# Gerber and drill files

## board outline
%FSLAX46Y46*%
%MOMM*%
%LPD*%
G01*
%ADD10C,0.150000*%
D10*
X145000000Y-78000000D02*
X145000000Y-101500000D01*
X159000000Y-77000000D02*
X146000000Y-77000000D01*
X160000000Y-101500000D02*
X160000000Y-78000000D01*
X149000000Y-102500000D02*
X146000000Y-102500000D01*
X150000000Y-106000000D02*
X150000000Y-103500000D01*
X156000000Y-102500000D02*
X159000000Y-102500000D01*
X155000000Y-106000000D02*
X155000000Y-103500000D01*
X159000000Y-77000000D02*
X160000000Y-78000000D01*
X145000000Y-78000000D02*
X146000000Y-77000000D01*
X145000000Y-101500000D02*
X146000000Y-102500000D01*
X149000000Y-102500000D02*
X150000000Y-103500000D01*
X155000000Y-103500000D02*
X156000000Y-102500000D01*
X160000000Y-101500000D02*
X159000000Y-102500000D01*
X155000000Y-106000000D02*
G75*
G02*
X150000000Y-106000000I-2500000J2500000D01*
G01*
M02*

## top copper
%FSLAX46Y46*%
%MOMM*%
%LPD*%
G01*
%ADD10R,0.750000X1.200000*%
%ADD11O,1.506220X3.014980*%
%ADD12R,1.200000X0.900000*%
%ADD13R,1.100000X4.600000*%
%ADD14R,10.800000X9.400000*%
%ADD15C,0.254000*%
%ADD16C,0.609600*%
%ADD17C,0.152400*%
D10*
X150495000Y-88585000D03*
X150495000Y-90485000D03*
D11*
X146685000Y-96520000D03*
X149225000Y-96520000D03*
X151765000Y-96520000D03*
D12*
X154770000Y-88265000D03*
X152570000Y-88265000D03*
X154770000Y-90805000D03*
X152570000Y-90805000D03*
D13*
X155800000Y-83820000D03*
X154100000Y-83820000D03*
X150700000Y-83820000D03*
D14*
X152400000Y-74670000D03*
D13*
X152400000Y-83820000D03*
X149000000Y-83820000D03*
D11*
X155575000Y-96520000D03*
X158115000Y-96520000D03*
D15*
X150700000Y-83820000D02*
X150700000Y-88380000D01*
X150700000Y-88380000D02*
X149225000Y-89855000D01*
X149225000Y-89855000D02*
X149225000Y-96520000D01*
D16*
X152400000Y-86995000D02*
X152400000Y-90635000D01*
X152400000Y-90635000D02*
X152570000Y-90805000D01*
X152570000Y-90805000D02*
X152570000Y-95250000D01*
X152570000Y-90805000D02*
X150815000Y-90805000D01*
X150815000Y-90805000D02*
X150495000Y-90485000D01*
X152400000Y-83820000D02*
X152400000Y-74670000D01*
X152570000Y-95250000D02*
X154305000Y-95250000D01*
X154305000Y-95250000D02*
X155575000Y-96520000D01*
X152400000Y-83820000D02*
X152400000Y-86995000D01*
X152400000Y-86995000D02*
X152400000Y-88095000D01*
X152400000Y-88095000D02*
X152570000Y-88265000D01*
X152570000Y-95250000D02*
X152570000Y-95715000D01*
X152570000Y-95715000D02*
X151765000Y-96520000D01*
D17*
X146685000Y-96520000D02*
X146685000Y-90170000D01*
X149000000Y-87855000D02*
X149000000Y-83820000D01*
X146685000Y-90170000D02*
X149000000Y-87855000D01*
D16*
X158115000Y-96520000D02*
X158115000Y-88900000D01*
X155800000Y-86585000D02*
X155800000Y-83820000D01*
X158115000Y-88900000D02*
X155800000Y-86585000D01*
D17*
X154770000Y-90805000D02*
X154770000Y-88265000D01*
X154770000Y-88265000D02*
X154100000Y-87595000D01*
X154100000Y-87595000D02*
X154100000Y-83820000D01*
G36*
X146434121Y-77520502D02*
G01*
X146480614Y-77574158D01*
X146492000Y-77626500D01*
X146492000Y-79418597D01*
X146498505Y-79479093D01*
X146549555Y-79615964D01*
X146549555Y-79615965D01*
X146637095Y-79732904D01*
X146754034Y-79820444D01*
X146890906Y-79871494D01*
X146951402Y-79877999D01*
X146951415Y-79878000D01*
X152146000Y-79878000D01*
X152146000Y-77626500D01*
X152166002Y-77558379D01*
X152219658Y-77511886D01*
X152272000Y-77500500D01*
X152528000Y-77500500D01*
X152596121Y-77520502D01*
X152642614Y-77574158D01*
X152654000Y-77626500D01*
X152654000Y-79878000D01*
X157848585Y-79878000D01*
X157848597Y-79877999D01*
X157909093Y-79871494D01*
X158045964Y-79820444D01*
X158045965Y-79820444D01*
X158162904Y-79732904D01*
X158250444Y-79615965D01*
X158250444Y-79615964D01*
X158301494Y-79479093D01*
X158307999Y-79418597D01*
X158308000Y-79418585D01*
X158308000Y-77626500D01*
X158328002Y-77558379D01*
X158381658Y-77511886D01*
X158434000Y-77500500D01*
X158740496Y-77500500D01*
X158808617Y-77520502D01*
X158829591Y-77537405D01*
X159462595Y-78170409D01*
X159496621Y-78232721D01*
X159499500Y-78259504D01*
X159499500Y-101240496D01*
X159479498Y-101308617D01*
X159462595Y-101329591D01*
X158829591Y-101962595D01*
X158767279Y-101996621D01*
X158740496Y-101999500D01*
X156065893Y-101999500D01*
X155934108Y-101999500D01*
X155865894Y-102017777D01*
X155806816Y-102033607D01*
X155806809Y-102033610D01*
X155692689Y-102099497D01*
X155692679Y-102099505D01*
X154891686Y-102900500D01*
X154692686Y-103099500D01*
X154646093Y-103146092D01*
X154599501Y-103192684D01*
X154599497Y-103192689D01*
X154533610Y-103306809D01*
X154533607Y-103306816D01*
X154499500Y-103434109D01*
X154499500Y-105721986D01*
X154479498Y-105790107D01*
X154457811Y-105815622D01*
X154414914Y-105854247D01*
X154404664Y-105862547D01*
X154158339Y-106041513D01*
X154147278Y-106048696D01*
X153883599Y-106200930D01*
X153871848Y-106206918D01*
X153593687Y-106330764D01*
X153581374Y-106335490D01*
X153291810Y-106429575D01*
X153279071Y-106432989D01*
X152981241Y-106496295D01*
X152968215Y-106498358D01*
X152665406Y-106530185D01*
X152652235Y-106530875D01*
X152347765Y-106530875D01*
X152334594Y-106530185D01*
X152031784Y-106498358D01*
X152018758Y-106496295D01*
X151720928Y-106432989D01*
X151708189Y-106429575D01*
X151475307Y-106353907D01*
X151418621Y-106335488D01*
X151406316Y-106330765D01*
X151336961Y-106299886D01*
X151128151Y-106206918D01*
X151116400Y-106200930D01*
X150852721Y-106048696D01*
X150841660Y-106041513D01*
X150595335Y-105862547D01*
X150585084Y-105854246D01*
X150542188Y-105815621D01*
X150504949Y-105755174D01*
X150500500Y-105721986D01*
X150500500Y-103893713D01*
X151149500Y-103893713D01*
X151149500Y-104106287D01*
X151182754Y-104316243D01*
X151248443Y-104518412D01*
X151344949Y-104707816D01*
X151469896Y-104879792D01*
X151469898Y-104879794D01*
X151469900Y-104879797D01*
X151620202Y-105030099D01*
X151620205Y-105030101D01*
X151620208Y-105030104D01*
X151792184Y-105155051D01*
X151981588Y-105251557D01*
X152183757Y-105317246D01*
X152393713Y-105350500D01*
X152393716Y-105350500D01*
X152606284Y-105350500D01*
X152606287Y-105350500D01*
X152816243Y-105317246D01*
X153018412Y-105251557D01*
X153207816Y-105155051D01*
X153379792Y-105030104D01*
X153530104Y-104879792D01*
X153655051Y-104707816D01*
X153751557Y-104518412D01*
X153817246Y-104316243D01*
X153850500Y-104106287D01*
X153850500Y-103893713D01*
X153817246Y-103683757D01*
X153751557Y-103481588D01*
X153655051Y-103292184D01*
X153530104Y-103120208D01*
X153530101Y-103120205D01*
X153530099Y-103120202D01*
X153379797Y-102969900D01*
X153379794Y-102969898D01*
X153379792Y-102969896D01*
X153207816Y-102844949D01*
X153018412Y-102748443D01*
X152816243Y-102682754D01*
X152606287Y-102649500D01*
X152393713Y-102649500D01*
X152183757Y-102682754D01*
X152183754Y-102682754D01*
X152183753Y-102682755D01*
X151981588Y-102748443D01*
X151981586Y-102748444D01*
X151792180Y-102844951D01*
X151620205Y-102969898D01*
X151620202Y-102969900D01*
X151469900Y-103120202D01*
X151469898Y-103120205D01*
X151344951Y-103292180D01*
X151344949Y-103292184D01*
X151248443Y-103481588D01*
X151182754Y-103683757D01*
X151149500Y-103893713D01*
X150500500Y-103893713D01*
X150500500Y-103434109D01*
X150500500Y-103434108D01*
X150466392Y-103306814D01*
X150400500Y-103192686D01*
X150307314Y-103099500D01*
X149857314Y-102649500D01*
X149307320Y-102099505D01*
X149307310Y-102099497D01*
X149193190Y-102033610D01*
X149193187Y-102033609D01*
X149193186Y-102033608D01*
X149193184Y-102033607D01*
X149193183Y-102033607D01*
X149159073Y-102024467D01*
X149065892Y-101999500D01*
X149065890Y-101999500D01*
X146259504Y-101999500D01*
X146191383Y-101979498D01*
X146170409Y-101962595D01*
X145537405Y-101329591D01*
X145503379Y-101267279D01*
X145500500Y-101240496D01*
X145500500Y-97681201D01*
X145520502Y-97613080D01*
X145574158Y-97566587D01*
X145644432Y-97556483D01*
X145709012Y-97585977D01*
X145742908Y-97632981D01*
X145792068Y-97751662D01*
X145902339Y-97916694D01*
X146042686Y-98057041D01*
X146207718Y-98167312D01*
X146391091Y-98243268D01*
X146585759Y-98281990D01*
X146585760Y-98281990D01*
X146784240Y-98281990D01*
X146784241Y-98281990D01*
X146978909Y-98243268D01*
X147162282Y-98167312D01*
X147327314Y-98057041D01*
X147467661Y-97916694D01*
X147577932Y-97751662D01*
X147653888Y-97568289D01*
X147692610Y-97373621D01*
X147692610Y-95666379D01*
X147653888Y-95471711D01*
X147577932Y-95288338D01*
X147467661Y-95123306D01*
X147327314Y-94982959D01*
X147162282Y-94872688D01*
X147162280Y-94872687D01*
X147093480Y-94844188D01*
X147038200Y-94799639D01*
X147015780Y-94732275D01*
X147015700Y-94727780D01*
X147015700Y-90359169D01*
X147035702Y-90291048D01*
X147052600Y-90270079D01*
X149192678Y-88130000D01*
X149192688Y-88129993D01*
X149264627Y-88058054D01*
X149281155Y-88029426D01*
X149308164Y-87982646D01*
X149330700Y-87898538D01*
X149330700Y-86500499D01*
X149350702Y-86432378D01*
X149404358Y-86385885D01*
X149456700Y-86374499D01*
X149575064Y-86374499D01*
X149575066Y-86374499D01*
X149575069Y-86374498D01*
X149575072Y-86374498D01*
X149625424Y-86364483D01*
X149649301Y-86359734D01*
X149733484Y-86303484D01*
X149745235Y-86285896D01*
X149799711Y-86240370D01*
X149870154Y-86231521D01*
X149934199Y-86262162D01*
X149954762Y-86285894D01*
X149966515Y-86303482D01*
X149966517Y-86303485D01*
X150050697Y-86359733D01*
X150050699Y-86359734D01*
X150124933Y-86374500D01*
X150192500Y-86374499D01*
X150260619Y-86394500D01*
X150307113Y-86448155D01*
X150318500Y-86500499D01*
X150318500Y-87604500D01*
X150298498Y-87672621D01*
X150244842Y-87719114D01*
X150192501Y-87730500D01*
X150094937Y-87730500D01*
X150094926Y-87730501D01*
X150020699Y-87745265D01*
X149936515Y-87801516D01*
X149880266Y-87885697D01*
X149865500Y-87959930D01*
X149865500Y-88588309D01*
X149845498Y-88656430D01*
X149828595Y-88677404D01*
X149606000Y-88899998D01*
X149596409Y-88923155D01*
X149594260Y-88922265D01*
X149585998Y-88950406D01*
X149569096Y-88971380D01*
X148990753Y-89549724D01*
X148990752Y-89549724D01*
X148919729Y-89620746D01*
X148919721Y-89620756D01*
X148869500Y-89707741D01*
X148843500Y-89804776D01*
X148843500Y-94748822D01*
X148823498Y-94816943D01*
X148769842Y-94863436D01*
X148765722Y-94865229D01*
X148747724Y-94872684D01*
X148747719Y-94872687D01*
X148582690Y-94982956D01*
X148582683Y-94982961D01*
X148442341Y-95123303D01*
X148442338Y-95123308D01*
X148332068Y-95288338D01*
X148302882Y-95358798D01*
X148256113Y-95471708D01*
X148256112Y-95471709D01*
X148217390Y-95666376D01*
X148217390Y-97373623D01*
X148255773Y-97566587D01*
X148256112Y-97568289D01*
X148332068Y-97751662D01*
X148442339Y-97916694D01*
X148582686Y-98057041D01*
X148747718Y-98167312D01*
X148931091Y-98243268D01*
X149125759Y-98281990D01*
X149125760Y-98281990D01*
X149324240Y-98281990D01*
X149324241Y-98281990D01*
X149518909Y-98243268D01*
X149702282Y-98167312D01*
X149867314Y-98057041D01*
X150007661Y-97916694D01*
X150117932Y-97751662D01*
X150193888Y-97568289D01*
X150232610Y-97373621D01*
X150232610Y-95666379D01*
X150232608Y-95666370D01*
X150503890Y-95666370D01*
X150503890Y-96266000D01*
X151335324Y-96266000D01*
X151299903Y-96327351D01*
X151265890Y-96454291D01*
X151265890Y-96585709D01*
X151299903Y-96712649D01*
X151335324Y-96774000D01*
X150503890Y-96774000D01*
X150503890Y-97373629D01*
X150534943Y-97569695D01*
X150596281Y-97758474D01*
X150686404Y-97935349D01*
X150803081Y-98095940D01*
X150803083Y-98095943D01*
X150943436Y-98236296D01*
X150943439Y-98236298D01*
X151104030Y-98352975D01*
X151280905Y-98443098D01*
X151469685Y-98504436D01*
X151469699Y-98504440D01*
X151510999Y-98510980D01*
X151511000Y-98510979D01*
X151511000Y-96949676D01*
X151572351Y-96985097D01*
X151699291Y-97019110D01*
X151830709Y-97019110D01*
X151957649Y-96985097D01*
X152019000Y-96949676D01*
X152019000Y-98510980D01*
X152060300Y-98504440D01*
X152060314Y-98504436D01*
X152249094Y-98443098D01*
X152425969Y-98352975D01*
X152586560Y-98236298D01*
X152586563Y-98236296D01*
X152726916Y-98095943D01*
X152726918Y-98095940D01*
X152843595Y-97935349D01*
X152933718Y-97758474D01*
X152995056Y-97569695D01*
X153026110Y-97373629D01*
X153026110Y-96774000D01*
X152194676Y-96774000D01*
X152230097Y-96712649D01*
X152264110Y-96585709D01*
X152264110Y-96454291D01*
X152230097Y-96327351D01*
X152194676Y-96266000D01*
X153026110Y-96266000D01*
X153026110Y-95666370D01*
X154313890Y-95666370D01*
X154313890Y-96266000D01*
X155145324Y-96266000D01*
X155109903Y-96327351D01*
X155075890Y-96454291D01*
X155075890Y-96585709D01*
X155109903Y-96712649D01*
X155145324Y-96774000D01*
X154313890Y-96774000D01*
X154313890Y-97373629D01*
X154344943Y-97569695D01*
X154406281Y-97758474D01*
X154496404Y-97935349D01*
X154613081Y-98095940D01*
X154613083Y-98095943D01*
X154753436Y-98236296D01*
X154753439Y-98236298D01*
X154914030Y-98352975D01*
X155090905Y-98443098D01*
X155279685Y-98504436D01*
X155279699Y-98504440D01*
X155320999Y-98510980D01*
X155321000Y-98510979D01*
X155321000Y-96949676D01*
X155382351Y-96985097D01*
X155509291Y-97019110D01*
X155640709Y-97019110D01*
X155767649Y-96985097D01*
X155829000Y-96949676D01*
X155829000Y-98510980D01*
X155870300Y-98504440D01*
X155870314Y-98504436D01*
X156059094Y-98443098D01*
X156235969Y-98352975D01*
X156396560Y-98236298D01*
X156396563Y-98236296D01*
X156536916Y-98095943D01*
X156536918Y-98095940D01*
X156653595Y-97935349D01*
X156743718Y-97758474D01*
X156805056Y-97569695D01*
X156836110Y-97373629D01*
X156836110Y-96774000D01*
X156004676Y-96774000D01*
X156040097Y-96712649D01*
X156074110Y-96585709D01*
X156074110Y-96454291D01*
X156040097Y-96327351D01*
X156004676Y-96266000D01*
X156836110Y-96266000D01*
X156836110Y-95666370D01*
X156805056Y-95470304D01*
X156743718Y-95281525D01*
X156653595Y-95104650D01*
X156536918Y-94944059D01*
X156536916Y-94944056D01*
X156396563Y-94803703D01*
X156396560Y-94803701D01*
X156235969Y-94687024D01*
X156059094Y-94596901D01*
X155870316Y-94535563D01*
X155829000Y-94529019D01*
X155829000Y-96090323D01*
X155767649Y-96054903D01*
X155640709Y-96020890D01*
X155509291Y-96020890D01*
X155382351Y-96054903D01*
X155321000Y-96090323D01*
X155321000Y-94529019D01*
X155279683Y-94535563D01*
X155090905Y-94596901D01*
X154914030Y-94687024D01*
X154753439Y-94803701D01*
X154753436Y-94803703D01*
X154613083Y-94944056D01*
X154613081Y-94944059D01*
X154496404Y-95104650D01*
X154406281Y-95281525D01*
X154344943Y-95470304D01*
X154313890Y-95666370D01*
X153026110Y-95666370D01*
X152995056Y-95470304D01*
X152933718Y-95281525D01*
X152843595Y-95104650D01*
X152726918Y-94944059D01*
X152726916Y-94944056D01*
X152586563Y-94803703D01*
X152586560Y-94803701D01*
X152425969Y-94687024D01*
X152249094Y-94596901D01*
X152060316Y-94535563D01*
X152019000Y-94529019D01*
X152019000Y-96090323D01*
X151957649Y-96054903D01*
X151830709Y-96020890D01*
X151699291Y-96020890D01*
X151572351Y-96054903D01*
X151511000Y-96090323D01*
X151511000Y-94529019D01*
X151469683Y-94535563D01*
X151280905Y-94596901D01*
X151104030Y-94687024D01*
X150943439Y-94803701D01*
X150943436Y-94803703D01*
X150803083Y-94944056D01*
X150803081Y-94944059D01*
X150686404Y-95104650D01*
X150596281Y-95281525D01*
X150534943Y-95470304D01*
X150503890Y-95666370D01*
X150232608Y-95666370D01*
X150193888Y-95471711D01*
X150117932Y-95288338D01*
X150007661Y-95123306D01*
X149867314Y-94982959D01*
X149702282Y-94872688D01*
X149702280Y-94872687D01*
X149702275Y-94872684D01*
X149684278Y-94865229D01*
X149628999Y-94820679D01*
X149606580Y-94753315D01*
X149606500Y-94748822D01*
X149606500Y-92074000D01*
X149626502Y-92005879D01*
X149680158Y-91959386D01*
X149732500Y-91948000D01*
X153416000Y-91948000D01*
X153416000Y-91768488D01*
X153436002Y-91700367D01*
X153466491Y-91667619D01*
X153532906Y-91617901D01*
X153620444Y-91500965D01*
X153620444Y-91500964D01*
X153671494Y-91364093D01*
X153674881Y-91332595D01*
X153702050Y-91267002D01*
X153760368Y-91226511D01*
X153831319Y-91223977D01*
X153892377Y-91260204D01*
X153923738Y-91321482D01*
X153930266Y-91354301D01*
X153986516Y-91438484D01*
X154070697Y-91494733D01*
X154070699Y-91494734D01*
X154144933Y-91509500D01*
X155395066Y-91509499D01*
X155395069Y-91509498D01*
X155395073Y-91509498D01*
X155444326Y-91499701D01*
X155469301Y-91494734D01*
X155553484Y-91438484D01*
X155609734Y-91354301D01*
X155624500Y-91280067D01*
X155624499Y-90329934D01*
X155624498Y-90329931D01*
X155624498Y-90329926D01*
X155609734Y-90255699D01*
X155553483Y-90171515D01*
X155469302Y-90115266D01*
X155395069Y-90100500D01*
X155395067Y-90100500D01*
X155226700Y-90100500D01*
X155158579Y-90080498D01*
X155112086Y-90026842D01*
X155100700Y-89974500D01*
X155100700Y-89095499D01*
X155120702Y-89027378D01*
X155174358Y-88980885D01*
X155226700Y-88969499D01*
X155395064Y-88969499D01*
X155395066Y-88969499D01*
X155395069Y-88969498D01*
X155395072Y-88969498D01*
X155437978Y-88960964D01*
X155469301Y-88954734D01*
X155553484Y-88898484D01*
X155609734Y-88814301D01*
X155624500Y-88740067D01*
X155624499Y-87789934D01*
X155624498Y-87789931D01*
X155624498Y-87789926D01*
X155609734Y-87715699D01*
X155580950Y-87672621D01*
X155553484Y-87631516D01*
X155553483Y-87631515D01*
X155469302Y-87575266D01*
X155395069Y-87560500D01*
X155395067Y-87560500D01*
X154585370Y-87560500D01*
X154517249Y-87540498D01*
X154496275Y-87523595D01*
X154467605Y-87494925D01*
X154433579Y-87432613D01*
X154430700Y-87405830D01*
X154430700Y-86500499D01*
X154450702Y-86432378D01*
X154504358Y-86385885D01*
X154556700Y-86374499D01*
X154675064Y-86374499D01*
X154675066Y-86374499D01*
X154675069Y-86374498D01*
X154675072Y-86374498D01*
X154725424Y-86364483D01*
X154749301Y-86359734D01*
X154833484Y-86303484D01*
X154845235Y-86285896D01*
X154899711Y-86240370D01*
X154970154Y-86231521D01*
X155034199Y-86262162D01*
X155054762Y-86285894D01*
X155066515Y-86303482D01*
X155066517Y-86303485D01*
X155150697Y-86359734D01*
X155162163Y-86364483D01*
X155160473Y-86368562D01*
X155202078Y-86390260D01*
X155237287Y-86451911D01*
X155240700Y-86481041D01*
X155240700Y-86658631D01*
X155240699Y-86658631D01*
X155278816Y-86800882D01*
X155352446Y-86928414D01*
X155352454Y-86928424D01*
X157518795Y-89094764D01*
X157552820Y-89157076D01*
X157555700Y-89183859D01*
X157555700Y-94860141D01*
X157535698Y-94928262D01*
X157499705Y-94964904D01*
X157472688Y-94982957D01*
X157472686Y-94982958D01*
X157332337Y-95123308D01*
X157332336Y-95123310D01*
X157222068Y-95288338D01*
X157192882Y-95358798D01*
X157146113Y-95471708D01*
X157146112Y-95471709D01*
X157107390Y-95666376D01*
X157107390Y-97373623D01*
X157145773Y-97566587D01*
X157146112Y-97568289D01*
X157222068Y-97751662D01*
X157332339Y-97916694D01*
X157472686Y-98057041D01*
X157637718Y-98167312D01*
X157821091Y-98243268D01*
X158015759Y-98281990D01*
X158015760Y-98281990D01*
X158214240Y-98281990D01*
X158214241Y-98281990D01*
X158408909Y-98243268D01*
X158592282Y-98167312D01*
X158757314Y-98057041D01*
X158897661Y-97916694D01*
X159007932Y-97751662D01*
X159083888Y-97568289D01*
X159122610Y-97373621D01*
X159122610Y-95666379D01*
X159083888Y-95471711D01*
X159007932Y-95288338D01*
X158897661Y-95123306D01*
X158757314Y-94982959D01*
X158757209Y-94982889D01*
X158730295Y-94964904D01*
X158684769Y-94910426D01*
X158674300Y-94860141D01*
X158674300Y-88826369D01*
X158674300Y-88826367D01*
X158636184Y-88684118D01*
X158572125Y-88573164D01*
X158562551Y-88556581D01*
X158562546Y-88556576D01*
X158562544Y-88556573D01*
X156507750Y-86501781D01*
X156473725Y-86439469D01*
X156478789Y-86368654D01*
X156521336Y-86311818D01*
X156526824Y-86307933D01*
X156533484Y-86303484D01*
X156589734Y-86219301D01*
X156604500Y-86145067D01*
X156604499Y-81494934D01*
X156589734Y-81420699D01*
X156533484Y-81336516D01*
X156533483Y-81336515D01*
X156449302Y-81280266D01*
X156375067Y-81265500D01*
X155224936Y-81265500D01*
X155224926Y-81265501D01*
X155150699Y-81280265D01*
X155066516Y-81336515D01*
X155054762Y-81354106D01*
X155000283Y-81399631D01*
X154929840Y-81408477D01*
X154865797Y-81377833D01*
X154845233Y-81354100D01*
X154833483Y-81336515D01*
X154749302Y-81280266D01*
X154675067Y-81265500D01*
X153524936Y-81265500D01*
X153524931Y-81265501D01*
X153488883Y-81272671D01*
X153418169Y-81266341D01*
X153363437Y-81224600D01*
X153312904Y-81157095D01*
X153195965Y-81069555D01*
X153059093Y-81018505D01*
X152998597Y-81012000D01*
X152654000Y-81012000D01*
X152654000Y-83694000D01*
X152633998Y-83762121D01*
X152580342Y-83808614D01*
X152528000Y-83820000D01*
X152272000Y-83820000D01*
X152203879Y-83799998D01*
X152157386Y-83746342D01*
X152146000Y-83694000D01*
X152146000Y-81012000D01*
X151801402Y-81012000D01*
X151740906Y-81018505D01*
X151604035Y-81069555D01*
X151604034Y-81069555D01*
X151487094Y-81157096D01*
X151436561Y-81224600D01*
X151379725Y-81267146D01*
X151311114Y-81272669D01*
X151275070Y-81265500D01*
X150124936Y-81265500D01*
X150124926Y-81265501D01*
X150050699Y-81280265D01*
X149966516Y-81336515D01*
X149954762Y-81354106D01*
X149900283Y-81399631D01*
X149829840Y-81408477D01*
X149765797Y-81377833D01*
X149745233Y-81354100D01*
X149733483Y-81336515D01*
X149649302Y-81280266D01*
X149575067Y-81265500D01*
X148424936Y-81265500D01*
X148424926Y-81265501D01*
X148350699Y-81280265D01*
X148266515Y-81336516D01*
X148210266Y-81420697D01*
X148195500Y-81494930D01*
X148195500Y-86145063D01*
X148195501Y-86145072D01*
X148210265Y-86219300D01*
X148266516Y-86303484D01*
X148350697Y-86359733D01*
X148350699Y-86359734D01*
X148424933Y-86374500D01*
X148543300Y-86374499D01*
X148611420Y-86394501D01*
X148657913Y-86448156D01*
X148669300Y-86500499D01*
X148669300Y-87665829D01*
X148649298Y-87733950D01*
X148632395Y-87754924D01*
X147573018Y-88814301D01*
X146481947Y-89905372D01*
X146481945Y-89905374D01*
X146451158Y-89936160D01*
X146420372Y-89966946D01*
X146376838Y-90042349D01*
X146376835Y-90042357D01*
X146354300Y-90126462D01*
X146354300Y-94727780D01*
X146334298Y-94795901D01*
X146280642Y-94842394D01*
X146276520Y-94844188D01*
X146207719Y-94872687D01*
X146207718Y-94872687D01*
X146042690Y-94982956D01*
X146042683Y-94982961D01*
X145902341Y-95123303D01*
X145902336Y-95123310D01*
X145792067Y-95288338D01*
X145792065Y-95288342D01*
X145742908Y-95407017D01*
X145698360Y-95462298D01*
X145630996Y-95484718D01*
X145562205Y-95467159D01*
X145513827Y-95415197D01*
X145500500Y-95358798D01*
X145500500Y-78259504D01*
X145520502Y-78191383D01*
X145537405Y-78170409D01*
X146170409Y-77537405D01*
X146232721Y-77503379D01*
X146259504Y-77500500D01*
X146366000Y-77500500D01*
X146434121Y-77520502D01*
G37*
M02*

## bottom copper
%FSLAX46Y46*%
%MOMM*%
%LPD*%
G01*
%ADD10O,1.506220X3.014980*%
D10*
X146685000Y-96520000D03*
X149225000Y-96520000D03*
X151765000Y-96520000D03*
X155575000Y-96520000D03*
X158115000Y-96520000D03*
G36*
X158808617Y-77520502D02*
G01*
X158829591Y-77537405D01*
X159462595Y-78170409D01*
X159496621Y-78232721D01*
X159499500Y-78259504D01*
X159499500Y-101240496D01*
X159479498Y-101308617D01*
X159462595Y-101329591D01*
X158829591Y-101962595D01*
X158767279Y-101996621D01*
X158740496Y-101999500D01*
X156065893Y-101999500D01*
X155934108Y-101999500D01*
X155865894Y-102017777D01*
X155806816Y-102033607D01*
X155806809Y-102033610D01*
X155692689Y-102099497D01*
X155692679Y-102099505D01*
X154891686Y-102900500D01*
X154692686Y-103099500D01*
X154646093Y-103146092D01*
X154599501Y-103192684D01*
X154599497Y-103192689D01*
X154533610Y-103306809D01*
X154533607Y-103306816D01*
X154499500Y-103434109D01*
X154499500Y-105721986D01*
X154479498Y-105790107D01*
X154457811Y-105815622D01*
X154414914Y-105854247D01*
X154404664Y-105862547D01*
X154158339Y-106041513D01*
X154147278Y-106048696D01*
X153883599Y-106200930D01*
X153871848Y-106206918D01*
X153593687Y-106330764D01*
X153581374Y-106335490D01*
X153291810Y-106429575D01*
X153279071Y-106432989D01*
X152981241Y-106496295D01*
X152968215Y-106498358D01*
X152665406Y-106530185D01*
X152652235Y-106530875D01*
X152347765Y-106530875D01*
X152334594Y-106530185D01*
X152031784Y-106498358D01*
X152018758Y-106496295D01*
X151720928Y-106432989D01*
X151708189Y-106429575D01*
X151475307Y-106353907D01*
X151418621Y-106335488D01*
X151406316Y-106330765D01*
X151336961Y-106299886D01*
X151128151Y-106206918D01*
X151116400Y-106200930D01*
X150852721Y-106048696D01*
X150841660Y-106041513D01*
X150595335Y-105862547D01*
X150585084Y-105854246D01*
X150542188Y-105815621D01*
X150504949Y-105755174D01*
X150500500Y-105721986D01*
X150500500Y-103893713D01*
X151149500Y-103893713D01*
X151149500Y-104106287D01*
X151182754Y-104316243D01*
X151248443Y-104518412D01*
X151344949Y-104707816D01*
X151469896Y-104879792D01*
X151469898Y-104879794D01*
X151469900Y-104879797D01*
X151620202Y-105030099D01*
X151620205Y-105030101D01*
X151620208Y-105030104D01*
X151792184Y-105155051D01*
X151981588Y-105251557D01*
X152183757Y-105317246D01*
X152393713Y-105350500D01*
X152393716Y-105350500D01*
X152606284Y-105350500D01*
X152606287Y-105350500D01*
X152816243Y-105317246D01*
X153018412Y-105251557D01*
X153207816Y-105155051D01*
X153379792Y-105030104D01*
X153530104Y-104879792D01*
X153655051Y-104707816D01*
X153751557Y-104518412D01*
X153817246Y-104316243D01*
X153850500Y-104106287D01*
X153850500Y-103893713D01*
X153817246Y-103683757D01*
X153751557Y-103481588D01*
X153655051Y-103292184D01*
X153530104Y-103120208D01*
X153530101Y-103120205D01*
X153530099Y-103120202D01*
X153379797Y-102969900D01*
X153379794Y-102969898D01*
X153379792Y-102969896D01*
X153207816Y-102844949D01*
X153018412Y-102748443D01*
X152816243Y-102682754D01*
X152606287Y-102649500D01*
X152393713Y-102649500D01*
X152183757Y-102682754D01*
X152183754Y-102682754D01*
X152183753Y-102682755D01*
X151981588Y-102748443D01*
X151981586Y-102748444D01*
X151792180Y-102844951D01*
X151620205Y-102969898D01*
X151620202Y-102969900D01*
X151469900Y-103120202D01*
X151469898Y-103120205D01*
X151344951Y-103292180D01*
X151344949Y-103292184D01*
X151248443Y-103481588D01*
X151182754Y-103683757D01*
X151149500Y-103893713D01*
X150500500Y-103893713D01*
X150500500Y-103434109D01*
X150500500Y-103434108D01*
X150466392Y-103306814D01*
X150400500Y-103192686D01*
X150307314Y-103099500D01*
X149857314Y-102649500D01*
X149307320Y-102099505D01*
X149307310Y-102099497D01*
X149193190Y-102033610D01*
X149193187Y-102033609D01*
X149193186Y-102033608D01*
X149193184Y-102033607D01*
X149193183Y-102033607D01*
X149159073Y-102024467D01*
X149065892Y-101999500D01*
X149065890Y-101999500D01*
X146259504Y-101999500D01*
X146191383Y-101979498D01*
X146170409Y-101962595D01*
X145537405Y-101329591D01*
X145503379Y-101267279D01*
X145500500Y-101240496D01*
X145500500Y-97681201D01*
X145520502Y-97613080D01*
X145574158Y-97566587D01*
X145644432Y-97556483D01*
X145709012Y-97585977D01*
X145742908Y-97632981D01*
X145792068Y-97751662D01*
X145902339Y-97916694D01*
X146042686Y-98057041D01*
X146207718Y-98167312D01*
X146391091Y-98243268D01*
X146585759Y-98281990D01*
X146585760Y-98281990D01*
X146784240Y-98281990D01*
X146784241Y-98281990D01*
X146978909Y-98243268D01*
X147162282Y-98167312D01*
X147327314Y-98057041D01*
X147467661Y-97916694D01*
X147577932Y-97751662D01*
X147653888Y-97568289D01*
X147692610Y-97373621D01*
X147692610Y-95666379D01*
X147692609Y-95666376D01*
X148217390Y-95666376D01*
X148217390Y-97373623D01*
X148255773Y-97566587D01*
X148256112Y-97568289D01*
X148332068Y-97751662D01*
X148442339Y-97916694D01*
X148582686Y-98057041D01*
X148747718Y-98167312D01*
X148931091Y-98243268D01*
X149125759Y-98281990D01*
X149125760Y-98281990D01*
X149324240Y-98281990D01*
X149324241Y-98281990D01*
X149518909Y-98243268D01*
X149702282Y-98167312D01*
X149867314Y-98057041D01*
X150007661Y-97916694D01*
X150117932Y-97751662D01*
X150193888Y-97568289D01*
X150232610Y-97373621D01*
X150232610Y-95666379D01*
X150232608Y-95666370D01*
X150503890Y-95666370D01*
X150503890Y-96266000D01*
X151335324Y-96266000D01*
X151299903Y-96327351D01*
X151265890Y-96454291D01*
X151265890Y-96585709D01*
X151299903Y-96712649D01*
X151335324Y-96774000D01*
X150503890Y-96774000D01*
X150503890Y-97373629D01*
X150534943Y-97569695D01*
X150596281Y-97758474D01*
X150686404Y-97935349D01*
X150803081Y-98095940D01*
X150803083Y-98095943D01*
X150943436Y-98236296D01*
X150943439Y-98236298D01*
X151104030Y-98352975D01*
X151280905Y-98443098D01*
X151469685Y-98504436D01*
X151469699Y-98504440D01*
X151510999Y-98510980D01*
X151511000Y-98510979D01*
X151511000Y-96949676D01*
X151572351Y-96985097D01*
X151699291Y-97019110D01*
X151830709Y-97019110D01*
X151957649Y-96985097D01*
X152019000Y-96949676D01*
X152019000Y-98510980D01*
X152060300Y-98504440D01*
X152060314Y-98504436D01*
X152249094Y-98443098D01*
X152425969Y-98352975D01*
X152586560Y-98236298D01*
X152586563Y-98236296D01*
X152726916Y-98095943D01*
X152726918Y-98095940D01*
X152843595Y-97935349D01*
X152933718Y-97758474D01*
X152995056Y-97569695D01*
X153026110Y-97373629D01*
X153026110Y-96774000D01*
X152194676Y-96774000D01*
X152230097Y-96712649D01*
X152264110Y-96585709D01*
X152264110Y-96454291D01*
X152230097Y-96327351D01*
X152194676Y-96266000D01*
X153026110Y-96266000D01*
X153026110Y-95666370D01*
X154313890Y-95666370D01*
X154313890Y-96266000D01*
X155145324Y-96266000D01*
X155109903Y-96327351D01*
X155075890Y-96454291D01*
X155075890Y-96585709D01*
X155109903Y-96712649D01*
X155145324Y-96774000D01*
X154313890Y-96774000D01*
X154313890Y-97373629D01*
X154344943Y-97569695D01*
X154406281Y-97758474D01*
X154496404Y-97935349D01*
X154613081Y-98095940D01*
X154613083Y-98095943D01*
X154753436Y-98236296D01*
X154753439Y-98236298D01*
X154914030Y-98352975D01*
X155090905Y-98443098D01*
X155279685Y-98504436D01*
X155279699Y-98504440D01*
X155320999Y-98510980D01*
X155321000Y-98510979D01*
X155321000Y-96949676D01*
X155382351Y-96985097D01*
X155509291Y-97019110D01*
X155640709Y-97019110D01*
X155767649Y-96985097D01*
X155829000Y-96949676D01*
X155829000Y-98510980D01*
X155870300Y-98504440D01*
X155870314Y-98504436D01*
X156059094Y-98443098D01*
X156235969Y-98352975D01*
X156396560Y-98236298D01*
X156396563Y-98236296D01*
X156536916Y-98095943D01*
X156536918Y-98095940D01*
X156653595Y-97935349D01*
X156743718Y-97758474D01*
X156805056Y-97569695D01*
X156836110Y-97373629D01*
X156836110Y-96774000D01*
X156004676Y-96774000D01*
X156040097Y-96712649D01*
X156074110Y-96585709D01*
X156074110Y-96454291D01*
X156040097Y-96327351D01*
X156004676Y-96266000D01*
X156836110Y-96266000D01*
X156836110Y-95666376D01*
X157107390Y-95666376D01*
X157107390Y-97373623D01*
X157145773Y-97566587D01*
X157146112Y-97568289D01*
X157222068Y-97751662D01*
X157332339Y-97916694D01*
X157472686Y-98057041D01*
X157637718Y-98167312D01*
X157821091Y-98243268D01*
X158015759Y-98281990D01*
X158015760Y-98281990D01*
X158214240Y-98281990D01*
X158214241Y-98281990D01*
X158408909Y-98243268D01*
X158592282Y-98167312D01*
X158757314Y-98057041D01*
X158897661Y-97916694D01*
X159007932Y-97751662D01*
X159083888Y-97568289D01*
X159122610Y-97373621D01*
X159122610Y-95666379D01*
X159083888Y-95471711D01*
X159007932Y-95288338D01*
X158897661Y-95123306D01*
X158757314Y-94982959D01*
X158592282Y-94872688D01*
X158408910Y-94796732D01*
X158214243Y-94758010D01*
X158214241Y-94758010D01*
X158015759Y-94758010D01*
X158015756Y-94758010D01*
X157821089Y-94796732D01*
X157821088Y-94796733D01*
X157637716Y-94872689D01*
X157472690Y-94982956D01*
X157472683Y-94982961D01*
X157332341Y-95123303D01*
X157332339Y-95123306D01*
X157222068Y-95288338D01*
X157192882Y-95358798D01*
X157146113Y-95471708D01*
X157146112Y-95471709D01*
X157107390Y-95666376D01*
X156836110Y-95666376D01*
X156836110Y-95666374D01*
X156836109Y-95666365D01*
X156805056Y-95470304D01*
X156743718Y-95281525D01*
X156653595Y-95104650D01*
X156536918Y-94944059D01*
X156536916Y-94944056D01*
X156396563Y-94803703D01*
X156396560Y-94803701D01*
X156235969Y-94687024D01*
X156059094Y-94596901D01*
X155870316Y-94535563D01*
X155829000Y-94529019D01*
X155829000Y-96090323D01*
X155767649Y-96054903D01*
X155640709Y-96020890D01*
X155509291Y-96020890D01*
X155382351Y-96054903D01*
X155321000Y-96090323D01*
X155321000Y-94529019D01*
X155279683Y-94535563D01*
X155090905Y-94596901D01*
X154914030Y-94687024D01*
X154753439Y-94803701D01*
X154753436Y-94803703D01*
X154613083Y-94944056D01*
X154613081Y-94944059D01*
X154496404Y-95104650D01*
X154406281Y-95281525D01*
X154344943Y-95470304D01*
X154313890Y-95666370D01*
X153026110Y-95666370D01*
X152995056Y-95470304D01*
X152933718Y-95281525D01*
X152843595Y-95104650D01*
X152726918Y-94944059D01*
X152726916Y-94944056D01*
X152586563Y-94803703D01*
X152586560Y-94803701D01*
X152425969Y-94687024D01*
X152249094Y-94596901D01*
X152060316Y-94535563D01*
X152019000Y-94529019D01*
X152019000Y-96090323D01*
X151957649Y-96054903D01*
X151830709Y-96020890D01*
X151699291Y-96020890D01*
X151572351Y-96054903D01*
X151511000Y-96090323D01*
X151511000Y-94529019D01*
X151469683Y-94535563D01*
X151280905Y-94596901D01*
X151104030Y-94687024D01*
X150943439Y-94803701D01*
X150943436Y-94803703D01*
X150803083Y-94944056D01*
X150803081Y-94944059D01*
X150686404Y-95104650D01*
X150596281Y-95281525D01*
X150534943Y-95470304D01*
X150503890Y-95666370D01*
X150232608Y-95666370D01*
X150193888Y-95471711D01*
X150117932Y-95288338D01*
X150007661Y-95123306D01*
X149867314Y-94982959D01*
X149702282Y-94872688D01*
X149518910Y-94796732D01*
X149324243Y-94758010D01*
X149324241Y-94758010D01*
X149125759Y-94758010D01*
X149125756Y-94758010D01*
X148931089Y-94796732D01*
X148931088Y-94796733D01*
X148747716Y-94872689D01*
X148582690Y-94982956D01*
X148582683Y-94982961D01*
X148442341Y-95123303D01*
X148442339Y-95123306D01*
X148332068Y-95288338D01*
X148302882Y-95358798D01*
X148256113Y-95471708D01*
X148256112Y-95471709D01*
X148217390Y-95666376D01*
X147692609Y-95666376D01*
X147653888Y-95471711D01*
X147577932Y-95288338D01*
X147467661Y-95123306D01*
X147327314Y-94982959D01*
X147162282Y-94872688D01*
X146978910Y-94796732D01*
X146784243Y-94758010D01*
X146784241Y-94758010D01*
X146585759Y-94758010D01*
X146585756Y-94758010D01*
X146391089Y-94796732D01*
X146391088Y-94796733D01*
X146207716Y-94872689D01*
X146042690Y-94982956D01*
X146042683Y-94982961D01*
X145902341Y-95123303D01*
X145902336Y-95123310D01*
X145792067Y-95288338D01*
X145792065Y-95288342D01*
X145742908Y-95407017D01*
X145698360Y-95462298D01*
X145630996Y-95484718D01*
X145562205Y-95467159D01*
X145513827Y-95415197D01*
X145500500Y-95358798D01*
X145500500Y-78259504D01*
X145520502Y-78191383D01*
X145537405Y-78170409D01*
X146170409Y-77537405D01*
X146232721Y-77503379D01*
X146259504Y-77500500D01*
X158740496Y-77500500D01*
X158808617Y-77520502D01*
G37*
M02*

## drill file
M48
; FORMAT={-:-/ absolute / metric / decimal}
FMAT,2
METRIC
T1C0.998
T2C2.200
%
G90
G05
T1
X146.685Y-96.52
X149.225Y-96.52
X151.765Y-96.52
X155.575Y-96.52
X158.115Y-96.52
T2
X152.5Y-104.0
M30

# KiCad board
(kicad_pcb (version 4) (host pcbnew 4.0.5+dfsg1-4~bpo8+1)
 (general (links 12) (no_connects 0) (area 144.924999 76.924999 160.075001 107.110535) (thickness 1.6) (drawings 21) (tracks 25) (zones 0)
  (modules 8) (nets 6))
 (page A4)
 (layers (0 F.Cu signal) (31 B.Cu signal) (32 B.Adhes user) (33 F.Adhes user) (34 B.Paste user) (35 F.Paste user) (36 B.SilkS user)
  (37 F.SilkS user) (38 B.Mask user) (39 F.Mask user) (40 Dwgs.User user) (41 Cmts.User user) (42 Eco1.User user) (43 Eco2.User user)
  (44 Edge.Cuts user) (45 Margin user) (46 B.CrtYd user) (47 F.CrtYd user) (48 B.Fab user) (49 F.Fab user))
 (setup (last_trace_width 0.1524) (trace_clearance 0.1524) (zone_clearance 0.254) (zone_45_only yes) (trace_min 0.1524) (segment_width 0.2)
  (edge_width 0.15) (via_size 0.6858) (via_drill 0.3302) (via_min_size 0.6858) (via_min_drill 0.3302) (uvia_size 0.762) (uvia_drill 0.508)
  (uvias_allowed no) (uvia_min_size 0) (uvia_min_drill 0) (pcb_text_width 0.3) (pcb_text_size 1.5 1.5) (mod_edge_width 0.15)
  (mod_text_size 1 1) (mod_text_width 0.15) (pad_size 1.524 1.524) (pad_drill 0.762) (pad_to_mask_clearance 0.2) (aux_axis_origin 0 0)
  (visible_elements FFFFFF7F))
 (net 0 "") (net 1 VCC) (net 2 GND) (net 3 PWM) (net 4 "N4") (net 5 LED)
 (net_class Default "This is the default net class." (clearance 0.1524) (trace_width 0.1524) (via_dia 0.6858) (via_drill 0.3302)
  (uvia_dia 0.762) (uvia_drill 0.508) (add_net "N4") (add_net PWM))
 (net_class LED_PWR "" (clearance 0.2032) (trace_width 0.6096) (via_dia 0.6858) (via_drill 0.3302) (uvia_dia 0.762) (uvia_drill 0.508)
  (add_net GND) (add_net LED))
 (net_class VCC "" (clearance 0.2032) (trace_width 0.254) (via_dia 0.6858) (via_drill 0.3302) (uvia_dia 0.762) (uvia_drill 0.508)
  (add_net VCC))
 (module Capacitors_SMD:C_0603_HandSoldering (layer F.Cu) (at 150.495 89.535 270)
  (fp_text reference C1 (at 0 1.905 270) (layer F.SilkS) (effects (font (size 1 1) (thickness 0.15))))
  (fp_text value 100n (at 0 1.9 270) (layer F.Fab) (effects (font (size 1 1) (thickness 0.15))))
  (pad 1 smd rect (at -0.95 0 270) (size 1.2 0.75) (layers F.Cu F.Paste F.Mask) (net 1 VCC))
  (pad 2 smd rect (at 0.95 0 270) (size 1.2 0.75) (layers F.Cu F.Paste F.Mask) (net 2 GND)))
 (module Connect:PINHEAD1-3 (layer F.Cu) (at 149.225 96.52)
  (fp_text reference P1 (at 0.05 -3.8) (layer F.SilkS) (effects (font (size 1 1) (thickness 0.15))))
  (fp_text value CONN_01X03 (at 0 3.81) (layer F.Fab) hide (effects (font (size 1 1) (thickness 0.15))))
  (pad 1 thru_hole oval (at -2.54 0) (size 1.50622 3.01498) (drill 0.99822) (layers *.Cu *.Mask) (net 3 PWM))
  (pad 2 thru_hole oval (at 0 0) (size 1.50622 3.01498) (drill 0.99822) (layers *.Cu *.Mask) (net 1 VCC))
  (pad 3 thru_hole oval (at 2.54 0) (size 1.50622 3.01498) (drill 0.99822) (layers *.Cu *.Mask) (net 2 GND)))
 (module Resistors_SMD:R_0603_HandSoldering (layer F.Cu) (at 153.67 88.265 180)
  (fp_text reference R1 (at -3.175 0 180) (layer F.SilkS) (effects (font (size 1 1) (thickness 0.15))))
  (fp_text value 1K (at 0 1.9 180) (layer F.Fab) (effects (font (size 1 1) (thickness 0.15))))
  (pad 1 smd rect (at -1.1 0 180) (size 1.2 0.9) (layers F.Cu F.Paste F.Mask) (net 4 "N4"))
  (pad 2 smd rect (at 1.1 0 180) (size 1.2 0.9) (layers F.Cu F.Paste F.Mask) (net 2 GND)))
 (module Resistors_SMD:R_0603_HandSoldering (layer F.Cu) (at 153.67 90.805 180)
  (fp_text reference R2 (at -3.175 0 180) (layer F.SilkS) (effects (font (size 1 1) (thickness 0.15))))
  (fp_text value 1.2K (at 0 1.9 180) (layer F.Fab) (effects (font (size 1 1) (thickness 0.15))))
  (pad 1 smd rect (at -1.1 0 180) (size 1.2 0.9) (layers F.Cu F.Paste F.Mask) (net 4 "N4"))
  (pad 2 smd rect (at 1.1 0 180) (size 1.2 0.9) (layers F.Cu F.Paste F.Mask) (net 2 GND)))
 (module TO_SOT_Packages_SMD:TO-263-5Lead (layer F.Cu) (at 152.4 83.82 90)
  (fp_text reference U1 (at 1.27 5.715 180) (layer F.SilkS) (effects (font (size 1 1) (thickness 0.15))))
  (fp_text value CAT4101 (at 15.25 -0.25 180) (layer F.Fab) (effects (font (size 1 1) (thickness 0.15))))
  (pad 5 smd rect (at 0 3.4 90) (size 4.6 1.1) (layers F.Cu F.Paste F.Mask) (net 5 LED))
  (pad 4 smd rect (at 0 1.7 90) (size 4.6 1.1) (layers F.Cu F.Paste F.Mask) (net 4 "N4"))
  (pad 2 smd rect (at 0 -1.7 90) (size 4.6 1.1) (layers F.Cu F.Paste F.Mask) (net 1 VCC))
  (pad 3 smd rect (at 9.15 0 90) (size 9.4 10.8) (layers F.Cu F.Paste F.Mask) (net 2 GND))
  (pad 3 smd rect (at 0 0 90) (size 4.6 1.1) (layers F.Cu F.Paste F.Mask) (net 2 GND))
  (pad 1 smd rect (at 0 -3.4 90) (size 4.6 1.1) (layers F.Cu F.Paste F.Mask) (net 3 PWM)))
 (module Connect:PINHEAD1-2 (layer F.Cu) (at 156.845 96.52)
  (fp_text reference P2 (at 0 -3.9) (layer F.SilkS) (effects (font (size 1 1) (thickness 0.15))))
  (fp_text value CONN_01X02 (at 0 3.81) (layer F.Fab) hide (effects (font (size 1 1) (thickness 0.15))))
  (pad 1 thru_hole oval (at -1.27 0) (size 1.50622 3.01498) (drill 0.99822) (layers *.Cu *.Mask) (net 2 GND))
  (pad 2 thru_hole oval (at 1.27 0) (size 1.50622 3.01498) (drill 0.99822) (layers *.Cu *.Mask) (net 5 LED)))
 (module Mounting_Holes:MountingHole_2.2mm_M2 (layer F.Cu) (at 152.5 104)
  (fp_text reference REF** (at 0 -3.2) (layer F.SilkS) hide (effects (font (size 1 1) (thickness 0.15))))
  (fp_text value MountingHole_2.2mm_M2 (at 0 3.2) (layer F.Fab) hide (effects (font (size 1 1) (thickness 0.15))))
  (pad 1 np_thru_hole circle (at 0 0) (size 2.2 2.2) (drill 2.2) (layers *.Cu *.Mask)))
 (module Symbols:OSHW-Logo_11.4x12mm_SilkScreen (layer B.Cu) (at 152.4 86.36 180)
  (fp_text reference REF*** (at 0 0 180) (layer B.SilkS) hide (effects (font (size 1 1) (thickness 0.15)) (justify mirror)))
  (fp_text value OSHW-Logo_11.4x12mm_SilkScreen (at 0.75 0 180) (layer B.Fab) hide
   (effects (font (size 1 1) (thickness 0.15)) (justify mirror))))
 (gr_line (start 145 78) (end 145 101.5) (angle 90) (layer Edge.Cuts) (width 0.15))
 (gr_line (start 159 77) (end 146 77) (angle 90) (layer Edge.Cuts) (width 0.15))
 (gr_line (start 160 101.5) (end 160 78) (angle 90) (layer Edge.Cuts) (width 0.15))
 (gr_line (start 149 102.5) (end 146 102.5) (angle 90) (layer Edge.Cuts) (width 0.15))
 (gr_line (start 150 106) (end 150 103.5) (angle 90) (layer Edge.Cuts) (width 0.15))
 (gr_line (start 156 102.5) (end 159 102.5) (angle 90) (layer Edge.Cuts) (width 0.15))
 (gr_line (start 155 106) (end 155 103.5) (angle 90) (layer Edge.Cuts) (width 0.15))
 (gr_line (start 159 77) (end 160 78) (angle 90) (layer Edge.Cuts) (width 0.15))
 (gr_line (start 145 78) (end 146 77) (angle 90) (layer Edge.Cuts) (width 0.15))
 (gr_line (start 145 101.5) (end 146 102.5) (angle 90) (layer Edge.Cuts) (width 0.15))
 (gr_line (start 149 102.5) (end 150 103.5) (angle 90) (layer Edge.Cuts) (width 0.15))
 (gr_line (start 155 103.5) (end 156 102.5) (angle 90) (layer Edge.Cuts) (width 0.15))
 (gr_line (start 160 101.5) (end 159 102.5) (angle 90) (layer Edge.Cuts) (width 0.15))
 (gr_arc (start 152.5 103.5) (end 155 106) (angle 90) (layer Edge.Cuts) (width 0.15))
 (segment (start 150.7 83.82) (end 150.7 88.38) (width 0.254) (layer F.Cu) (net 1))
 (segment (start 150.7 88.38) (end 149.225 89.855) (width 0.254) (layer F.Cu) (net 1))
 (segment (start 149.225 89.855) (end 149.225 96.52) (width 0.254) (layer F.Cu) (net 1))
 (segment (start 152.4 86.995) (end 152.4 90.635) (width 0.6096) (layer F.Cu) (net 2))
 (segment (start 152.4 90.635) (end 152.57 90.805) (width 0.6096) (layer F.Cu) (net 2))
 (segment (start 152.57 90.805) (end 152.57 95.25) (width 0.6096) (layer F.Cu) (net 2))
 (segment (start 152.57 90.805) (end 150.815 90.805) (width 0.6096) (layer F.Cu) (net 2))
 (segment (start 150.815 90.805) (end 150.495 90.485) (width 0.6096) (layer F.Cu) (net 2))
 (segment (start 152.4 83.82) (end 152.4 74.67) (width 0.6096) (layer F.Cu) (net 2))
 (segment (start 152.57 95.25) (end 154.305 95.25) (width 0.6096) (layer F.Cu) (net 2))
 (segment (start 154.305 95.25) (end 155.575 96.52) (width 0.6096) (layer F.Cu) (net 2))
 (segment (start 152.4 83.82) (end 152.4 86.995) (width 0.6096) (layer F.Cu) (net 2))
 (segment (start 152.4 86.995) (end 152.4 88.095) (width 0.6096) (layer F.Cu) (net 2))
 (segment (start 152.4 88.095) (end 152.57 88.265) (width 0.6096) (layer F.Cu) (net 2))
 (segment (start 152.57 95.25) (end 152.57 95.715) (width 0.6096) (layer F.Cu) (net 2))
 (segment (start 152.57 95.715) (end 151.765 96.52) (width 0.6096) (layer F.Cu) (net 2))
 (segment (start 146.685 96.52) (end 146.685 90.17) (width 0.1524) (layer F.Cu) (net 3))
 (segment (start 149 87.855) (end 149 83.82) (width 0.1524) (layer F.Cu) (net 3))
 (segment (start 146.685 90.17) (end 149 87.855) (width 0.1524) (layer F.Cu) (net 3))
 (segment (start 158.115 96.52) (end 158.115 88.9) (width 0.6096) (layer F.Cu) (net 5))
 (segment (start 155.8 86.585) (end 155.8 83.82) (width 0.6096) (layer F.Cu) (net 5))
 (segment (start 158.115 88.9) (end 155.8 86.585) (width 0.6096) (layer F.Cu) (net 5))
 (segment (start 154.77 90.805) (end 154.77 88.265) (width 0.1524) (layer F.Cu) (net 4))
 (segment (start 154.77 88.265) (end 154.1 87.595) (width 0.1524) (layer F.Cu) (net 4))
 (segment (start 154.1 87.595) (end 154.1 83.82) (width 0.1524) (layer F.Cu) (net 4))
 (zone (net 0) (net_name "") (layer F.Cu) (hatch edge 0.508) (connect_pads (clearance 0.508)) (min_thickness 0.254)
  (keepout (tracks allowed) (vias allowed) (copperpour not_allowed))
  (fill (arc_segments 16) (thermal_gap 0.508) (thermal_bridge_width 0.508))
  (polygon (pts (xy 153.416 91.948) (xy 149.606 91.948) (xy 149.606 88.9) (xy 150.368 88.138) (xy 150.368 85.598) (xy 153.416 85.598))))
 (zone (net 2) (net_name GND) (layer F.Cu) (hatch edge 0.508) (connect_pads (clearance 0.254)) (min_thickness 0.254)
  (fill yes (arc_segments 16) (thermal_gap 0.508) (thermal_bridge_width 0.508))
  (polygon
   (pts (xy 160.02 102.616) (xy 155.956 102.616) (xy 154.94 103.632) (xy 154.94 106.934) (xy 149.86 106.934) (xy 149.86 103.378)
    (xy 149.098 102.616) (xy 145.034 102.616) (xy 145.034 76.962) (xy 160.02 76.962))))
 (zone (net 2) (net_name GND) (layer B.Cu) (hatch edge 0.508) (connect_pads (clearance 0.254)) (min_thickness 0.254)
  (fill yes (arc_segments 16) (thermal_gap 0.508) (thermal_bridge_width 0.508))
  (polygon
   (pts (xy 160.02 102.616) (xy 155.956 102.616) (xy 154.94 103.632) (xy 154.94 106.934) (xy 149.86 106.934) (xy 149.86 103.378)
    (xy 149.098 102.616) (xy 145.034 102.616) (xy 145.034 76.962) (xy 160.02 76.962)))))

